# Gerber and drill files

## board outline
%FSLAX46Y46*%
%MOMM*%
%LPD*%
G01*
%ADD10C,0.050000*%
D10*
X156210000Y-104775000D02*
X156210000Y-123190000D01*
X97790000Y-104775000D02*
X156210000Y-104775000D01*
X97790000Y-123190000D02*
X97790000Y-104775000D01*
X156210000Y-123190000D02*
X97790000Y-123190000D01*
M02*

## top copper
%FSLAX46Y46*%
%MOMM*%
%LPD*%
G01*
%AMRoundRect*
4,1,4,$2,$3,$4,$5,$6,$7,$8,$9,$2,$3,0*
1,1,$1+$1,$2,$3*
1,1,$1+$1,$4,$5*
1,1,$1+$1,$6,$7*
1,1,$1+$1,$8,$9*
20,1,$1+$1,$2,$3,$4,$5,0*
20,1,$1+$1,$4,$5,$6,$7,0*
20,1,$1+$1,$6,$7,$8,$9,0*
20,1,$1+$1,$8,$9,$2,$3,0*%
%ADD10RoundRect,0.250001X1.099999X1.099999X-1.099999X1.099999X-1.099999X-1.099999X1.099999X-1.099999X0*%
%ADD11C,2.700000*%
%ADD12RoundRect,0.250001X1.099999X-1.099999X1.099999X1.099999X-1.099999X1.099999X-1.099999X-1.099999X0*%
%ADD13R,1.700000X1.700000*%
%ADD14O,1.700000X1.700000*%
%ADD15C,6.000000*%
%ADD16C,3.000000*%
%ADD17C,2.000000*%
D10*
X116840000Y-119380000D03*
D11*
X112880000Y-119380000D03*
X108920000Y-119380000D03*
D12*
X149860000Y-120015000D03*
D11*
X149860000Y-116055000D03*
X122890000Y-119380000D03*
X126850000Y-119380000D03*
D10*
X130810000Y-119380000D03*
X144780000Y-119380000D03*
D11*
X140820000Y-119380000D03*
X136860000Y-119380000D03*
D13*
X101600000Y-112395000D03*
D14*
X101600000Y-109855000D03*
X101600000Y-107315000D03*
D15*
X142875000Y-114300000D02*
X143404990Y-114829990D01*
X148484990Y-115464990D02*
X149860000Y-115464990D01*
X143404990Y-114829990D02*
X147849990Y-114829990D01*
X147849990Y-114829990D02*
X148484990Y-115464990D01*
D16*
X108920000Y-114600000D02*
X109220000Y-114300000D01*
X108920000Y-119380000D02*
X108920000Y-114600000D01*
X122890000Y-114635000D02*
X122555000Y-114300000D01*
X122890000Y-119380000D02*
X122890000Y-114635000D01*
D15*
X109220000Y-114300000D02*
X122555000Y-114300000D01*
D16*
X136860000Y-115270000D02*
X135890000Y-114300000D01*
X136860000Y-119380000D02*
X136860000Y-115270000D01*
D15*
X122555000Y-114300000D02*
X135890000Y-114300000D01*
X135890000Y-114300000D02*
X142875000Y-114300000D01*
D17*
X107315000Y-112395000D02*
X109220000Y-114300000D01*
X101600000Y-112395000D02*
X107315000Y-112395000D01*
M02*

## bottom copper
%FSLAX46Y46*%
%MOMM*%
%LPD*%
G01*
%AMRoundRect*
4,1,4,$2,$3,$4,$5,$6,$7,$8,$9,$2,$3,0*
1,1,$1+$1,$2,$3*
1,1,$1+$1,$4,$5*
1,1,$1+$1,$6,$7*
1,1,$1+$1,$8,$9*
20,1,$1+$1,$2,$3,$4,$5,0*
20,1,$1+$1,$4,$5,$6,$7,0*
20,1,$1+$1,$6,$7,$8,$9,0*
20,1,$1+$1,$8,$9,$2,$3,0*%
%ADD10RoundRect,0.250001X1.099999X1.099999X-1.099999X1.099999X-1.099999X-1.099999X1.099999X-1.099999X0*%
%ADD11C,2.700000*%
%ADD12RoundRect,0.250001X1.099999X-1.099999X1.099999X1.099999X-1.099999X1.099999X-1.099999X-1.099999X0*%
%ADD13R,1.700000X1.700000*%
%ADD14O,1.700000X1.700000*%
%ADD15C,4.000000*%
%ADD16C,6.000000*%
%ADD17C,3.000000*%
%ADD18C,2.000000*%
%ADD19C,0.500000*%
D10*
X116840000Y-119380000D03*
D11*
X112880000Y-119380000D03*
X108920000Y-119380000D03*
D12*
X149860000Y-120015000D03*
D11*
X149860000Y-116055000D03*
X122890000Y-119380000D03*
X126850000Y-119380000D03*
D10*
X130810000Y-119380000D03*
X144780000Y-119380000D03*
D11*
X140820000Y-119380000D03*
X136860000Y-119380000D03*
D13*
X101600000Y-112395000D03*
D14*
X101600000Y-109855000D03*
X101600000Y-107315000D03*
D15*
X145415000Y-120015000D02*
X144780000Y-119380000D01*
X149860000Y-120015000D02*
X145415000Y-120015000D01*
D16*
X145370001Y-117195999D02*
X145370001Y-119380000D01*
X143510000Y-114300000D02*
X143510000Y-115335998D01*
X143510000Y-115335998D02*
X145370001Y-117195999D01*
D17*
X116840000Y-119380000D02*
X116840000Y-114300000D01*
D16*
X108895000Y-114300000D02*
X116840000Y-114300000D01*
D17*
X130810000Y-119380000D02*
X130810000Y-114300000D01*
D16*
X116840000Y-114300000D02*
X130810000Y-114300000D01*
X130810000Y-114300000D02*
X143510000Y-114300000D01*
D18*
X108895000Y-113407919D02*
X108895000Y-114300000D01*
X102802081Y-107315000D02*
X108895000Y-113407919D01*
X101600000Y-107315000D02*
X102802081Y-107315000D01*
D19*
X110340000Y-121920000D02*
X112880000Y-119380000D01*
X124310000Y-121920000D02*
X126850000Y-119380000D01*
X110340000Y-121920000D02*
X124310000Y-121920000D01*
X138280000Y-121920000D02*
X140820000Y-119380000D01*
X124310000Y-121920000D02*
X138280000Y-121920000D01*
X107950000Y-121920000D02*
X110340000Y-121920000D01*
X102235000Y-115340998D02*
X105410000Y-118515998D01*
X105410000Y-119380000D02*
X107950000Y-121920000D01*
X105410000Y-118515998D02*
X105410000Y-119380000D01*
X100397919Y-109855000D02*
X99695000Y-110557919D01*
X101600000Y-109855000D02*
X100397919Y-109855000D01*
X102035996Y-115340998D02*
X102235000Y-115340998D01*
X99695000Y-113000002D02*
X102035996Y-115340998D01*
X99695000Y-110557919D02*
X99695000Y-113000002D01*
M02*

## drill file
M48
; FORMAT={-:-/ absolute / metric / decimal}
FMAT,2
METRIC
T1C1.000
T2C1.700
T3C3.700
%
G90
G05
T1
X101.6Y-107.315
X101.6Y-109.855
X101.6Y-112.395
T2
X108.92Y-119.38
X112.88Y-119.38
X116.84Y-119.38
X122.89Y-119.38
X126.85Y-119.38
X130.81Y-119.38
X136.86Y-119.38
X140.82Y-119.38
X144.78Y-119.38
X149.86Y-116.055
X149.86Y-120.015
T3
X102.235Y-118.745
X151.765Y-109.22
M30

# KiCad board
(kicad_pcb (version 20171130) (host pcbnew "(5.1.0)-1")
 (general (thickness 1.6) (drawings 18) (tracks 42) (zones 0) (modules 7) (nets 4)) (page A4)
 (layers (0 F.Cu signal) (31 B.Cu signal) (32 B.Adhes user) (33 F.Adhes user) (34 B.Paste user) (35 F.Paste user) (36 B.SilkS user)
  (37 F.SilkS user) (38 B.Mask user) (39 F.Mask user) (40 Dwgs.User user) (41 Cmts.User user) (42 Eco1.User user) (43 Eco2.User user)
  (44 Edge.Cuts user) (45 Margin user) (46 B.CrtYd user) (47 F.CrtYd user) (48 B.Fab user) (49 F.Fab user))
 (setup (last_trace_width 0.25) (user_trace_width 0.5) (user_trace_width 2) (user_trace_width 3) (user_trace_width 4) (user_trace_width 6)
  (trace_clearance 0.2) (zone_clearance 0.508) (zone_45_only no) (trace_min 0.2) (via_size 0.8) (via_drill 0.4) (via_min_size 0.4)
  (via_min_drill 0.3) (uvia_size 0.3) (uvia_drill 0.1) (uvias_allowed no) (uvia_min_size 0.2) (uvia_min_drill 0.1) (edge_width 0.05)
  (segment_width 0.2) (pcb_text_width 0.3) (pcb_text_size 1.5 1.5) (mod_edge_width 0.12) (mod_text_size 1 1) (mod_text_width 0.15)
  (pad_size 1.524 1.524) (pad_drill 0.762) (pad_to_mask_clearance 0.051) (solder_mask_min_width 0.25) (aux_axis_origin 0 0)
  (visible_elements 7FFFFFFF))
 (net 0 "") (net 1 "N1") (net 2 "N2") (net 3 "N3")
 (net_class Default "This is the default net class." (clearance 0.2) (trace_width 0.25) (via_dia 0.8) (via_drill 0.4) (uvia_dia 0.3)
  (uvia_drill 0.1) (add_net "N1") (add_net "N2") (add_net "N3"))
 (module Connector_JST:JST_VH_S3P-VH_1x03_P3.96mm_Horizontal (layer F.Cu) (at 116.84 119.38 180)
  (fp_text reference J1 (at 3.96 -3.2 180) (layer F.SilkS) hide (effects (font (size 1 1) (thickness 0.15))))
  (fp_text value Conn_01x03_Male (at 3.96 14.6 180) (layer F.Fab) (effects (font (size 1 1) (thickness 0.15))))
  (pad 1 thru_hole roundrect (at 0 0 180) (size 2.7 2.7) (drill 1.7) (layers *.Cu *.Mask) (roundrect_rratio 0.09259299999999999)
   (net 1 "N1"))
  (pad 2 thru_hole circle (at 3.96 0 180) (size 2.7 2.7) (drill 1.7) (layers *.Cu *.Mask) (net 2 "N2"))
  (pad 3 thru_hole circle (at 7.92 0 180) (size 2.7 2.7) (drill 1.7) (layers *.Cu *.Mask) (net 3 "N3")))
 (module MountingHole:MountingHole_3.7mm (layer F.Cu) (at 102.235 118.745)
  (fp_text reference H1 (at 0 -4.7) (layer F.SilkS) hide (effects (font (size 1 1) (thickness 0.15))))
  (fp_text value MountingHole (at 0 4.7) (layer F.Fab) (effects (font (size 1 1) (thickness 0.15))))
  (pad 1 np_thru_hole circle (at 0 0) (size 3.7 3.7) (drill 3.7) (layers *.Cu *.Mask)))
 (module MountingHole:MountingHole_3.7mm (layer F.Cu) (at 151.765 109.22)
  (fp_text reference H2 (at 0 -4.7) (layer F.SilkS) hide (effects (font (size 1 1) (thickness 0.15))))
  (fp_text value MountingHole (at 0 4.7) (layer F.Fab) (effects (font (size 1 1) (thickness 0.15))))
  (pad 1 np_thru_hole circle (at 0 0) (size 3.7 3.7) (drill 3.7) (layers *.Cu *.Mask)))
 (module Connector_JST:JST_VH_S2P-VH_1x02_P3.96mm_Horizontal (layer F.Cu) (at 149.86 120.015 90)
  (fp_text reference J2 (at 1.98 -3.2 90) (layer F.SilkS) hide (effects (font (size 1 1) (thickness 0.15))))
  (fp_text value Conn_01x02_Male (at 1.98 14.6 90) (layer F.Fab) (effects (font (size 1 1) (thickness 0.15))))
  (pad 1 thru_hole roundrect (at 0 0 90) (size 2.7 2.7) (drill 1.7) (layers *.Cu *.Mask) (roundrect_rratio 0.09259299999999999) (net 1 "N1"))
  (pad 2 thru_hole circle (at 3.96 0 90) (size 2.7 2.7) (drill 1.7) (layers *.Cu *.Mask) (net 3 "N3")))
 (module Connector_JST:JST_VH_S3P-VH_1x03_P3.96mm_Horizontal (layer F.Cu) (at 130.81 119.38 180)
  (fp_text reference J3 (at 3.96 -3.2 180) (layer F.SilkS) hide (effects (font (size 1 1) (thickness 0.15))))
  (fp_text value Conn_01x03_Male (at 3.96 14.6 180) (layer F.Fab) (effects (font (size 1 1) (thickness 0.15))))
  (pad 3 thru_hole circle (at 7.92 0 180) (size 2.7 2.7) (drill 1.7) (layers *.Cu *.Mask) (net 3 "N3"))
  (pad 2 thru_hole circle (at 3.96 0 180) (size 2.7 2.7) (drill 1.7) (layers *.Cu *.Mask) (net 2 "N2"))
  (pad 1 thru_hole roundrect (at 0 0 180) (size 2.7 2.7) (drill 1.7) (layers *.Cu *.Mask) (roundrect_rratio 0.09259299999999999)
   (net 1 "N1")))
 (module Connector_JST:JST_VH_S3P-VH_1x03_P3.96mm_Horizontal (layer F.Cu) (at 144.78 119.38 180)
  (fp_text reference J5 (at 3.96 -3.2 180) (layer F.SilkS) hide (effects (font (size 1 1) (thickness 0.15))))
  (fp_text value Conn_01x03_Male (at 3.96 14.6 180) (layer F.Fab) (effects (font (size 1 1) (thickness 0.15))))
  (pad 1 thru_hole roundrect (at 0 0 180) (size 2.7 2.7) (drill 1.7) (layers *.Cu *.Mask) (roundrect_rratio 0.09259299999999999)
   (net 1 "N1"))
  (pad 2 thru_hole circle (at 3.96 0 180) (size 2.7 2.7) (drill 1.7) (layers *.Cu *.Mask) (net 2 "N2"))
  (pad 3 thru_hole circle (at 7.92 0 180) (size 2.7 2.7) (drill 1.7) (layers *.Cu *.Mask) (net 3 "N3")))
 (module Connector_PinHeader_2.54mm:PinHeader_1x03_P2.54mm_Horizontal (layer F.Cu) (at 101.6 112.395 180)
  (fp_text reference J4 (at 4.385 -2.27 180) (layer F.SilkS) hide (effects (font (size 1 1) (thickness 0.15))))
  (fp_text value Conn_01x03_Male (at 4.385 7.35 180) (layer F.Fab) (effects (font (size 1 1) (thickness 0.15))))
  (pad 1 thru_hole rect (at 0 0 180) (size 1.7 1.7) (drill 1) (layers *.Cu *.Mask) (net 3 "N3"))
  (pad 2 thru_hole oval (at 0 2.54 180) (size 1.7 1.7) (drill 1) (layers *.Cu *.Mask) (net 2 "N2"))
  (pad 3 thru_hole oval (at 0 5.08 180) (size 1.7 1.7) (drill 1) (layers *.Cu *.Mask) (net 1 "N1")))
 (gr_line (start 156.21 104.775) (end 156.21 123.19) (layer Edge.Cuts) (width 0.05))
 (gr_line (start 97.79 104.775) (end 156.21 104.775) (layer Edge.Cuts) (width 0.05))
 (gr_line (start 97.79 123.19) (end 97.79 104.775) (layer Edge.Cuts) (width 0.05))
 (gr_line (start 156.21 123.19) (end 97.79 123.19) (layer Edge.Cuts) (width 0.05))
 (segment (start 145.415 120.015) (end 144.78 119.38) (width 4) (layer B.Cu) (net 1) (status 30))
 (segment (start 149.86 120.015) (end 145.415 120.015) (width 4) (layer B.Cu) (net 1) (status 30))
 (segment (start 145.370001 117.195999) (end 145.370001 119.38) (width 6) (layer B.Cu) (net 1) (status 20))
 (segment (start 143.51 114.3) (end 143.51 115.335998) (width 6) (layer B.Cu) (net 1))
 (segment (start 143.51 115.335998) (end 145.370001 117.195999) (width 6) (layer B.Cu) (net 1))
 (segment (start 116.84 119.38) (end 116.84 114.3) (width 3) (layer B.Cu) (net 1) (status 10))
 (segment (start 108.895 114.3) (end 116.84 114.3) (width 6) (layer B.Cu) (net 1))
 (segment (start 130.81 119.38) (end 130.81 114.3) (width 3) (layer B.Cu) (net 1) (status 10))
 (segment (start 116.84 114.3) (end 130.81 114.3) (width 6) (layer B.Cu) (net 1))
 (segment (start 130.81 114.3) (end 143.51 114.3) (width 6) (layer B.Cu) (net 1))
 (segment (start 108.895 113.407919) (end 108.895 114.3) (width 2) (layer B.Cu) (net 1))
 (segment (start 102.802081 107.315) (end 108.895 113.407919) (width 2) (layer B.Cu) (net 1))
 (segment (start 101.6 107.315) (end 102.802081 107.315) (width 2) (layer B.Cu) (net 1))
 (segment (start 110.34 121.92) (end 112.88 119.38) (width 0.5) (layer B.Cu) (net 2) (status 20))
 (segment (start 124.31 121.92) (end 126.85 119.38) (width 0.5) (layer B.Cu) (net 2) (status 20))
 (segment (start 110.34 121.92) (end 124.31 121.92) (width 0.5) (layer B.Cu) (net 2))
 (segment (start 138.28 121.92) (end 140.82 119.38) (width 0.5) (layer B.Cu) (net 2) (status 20))
 (segment (start 124.31 121.92) (end 138.28 121.92) (width 0.5) (layer B.Cu) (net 2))
 (segment (start 107.95 121.92) (end 110.34 121.92) (width 0.5) (layer B.Cu) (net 2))
 (segment (start 102.235 115.340998) (end 105.41 118.515998) (width 0.5) (layer B.Cu) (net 2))
 (segment (start 105.41 119.38) (end 107.95 121.92) (width 0.5) (layer B.Cu) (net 2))
 (segment (start 105.41 118.515998) (end 105.41 119.38) (width 0.5) (layer B.Cu) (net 2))
 (segment (start 100.397919 109.855) (end 99.695 110.557919) (width 0.5) (layer B.Cu) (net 2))
 (segment (start 101.6 109.855) (end 100.397919 109.855) (width 0.5) (layer B.Cu) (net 2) (status 10))
 (segment (start 102.035996 115.340998) (end 102.235 115.340998) (width 0.5) (layer B.Cu) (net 2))
 (segment (start 99.695 113.000002) (end 102.035996 115.340998) (width 0.5) (layer B.Cu) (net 2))
 (segment (start 99.695 110.557919) (end 99.695 113.000002) (width 0.5) (layer B.Cu) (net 2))
 (segment (start 142.875 114.3) (end 143.40499 114.82999) (width 6) (layer F.Cu) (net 3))
 (segment (start 148.48499 115.46499) (end 149.86 115.46499) (width 6) (layer F.Cu) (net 3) (status 20))
 (segment (start 143.40499 114.82999) (end 147.84999 114.82999) (width 6) (layer F.Cu) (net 3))
 (segment (start 147.84999 114.82999) (end 148.48499 115.46499) (width 6) (layer F.Cu) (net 3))
 (segment (start 108.92 114.6) (end 109.22 114.3) (width 3) (layer F.Cu) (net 3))
 (segment (start 108.92 119.38) (end 108.92 114.6) (width 3) (layer F.Cu) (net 3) (status 10))
 (segment (start 122.89 114.635) (end 122.555 114.3) (width 3) (layer F.Cu) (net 3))
 (segment (start 122.89 119.38) (end 122.89 114.635) (width 3) (layer F.Cu) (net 3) (status 10))
 (segment (start 109.22 114.3) (end 122.555 114.3) (width 6) (layer F.Cu) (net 3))
 (segment (start 136.86 115.27) (end 135.89 114.3) (width 3) (layer F.Cu) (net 3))
 (segment (start 136.86 119.38) (end 136.86 115.27) (width 3) (layer F.Cu) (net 3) (status 10))
 (segment (start 122.555 114.3) (end 135.89 114.3) (width 6) (layer F.Cu) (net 3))
 (segment (start 135.89 114.3) (end 142.875 114.3) (width 6) (layer F.Cu) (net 3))
 (segment (start 107.315 112.395) (end 109.22 114.3) (width 2) (layer F.Cu) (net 3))
 (segment (start 101.6 112.395) (end 107.315 112.395) (width 2) (layer F.Cu) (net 3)))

